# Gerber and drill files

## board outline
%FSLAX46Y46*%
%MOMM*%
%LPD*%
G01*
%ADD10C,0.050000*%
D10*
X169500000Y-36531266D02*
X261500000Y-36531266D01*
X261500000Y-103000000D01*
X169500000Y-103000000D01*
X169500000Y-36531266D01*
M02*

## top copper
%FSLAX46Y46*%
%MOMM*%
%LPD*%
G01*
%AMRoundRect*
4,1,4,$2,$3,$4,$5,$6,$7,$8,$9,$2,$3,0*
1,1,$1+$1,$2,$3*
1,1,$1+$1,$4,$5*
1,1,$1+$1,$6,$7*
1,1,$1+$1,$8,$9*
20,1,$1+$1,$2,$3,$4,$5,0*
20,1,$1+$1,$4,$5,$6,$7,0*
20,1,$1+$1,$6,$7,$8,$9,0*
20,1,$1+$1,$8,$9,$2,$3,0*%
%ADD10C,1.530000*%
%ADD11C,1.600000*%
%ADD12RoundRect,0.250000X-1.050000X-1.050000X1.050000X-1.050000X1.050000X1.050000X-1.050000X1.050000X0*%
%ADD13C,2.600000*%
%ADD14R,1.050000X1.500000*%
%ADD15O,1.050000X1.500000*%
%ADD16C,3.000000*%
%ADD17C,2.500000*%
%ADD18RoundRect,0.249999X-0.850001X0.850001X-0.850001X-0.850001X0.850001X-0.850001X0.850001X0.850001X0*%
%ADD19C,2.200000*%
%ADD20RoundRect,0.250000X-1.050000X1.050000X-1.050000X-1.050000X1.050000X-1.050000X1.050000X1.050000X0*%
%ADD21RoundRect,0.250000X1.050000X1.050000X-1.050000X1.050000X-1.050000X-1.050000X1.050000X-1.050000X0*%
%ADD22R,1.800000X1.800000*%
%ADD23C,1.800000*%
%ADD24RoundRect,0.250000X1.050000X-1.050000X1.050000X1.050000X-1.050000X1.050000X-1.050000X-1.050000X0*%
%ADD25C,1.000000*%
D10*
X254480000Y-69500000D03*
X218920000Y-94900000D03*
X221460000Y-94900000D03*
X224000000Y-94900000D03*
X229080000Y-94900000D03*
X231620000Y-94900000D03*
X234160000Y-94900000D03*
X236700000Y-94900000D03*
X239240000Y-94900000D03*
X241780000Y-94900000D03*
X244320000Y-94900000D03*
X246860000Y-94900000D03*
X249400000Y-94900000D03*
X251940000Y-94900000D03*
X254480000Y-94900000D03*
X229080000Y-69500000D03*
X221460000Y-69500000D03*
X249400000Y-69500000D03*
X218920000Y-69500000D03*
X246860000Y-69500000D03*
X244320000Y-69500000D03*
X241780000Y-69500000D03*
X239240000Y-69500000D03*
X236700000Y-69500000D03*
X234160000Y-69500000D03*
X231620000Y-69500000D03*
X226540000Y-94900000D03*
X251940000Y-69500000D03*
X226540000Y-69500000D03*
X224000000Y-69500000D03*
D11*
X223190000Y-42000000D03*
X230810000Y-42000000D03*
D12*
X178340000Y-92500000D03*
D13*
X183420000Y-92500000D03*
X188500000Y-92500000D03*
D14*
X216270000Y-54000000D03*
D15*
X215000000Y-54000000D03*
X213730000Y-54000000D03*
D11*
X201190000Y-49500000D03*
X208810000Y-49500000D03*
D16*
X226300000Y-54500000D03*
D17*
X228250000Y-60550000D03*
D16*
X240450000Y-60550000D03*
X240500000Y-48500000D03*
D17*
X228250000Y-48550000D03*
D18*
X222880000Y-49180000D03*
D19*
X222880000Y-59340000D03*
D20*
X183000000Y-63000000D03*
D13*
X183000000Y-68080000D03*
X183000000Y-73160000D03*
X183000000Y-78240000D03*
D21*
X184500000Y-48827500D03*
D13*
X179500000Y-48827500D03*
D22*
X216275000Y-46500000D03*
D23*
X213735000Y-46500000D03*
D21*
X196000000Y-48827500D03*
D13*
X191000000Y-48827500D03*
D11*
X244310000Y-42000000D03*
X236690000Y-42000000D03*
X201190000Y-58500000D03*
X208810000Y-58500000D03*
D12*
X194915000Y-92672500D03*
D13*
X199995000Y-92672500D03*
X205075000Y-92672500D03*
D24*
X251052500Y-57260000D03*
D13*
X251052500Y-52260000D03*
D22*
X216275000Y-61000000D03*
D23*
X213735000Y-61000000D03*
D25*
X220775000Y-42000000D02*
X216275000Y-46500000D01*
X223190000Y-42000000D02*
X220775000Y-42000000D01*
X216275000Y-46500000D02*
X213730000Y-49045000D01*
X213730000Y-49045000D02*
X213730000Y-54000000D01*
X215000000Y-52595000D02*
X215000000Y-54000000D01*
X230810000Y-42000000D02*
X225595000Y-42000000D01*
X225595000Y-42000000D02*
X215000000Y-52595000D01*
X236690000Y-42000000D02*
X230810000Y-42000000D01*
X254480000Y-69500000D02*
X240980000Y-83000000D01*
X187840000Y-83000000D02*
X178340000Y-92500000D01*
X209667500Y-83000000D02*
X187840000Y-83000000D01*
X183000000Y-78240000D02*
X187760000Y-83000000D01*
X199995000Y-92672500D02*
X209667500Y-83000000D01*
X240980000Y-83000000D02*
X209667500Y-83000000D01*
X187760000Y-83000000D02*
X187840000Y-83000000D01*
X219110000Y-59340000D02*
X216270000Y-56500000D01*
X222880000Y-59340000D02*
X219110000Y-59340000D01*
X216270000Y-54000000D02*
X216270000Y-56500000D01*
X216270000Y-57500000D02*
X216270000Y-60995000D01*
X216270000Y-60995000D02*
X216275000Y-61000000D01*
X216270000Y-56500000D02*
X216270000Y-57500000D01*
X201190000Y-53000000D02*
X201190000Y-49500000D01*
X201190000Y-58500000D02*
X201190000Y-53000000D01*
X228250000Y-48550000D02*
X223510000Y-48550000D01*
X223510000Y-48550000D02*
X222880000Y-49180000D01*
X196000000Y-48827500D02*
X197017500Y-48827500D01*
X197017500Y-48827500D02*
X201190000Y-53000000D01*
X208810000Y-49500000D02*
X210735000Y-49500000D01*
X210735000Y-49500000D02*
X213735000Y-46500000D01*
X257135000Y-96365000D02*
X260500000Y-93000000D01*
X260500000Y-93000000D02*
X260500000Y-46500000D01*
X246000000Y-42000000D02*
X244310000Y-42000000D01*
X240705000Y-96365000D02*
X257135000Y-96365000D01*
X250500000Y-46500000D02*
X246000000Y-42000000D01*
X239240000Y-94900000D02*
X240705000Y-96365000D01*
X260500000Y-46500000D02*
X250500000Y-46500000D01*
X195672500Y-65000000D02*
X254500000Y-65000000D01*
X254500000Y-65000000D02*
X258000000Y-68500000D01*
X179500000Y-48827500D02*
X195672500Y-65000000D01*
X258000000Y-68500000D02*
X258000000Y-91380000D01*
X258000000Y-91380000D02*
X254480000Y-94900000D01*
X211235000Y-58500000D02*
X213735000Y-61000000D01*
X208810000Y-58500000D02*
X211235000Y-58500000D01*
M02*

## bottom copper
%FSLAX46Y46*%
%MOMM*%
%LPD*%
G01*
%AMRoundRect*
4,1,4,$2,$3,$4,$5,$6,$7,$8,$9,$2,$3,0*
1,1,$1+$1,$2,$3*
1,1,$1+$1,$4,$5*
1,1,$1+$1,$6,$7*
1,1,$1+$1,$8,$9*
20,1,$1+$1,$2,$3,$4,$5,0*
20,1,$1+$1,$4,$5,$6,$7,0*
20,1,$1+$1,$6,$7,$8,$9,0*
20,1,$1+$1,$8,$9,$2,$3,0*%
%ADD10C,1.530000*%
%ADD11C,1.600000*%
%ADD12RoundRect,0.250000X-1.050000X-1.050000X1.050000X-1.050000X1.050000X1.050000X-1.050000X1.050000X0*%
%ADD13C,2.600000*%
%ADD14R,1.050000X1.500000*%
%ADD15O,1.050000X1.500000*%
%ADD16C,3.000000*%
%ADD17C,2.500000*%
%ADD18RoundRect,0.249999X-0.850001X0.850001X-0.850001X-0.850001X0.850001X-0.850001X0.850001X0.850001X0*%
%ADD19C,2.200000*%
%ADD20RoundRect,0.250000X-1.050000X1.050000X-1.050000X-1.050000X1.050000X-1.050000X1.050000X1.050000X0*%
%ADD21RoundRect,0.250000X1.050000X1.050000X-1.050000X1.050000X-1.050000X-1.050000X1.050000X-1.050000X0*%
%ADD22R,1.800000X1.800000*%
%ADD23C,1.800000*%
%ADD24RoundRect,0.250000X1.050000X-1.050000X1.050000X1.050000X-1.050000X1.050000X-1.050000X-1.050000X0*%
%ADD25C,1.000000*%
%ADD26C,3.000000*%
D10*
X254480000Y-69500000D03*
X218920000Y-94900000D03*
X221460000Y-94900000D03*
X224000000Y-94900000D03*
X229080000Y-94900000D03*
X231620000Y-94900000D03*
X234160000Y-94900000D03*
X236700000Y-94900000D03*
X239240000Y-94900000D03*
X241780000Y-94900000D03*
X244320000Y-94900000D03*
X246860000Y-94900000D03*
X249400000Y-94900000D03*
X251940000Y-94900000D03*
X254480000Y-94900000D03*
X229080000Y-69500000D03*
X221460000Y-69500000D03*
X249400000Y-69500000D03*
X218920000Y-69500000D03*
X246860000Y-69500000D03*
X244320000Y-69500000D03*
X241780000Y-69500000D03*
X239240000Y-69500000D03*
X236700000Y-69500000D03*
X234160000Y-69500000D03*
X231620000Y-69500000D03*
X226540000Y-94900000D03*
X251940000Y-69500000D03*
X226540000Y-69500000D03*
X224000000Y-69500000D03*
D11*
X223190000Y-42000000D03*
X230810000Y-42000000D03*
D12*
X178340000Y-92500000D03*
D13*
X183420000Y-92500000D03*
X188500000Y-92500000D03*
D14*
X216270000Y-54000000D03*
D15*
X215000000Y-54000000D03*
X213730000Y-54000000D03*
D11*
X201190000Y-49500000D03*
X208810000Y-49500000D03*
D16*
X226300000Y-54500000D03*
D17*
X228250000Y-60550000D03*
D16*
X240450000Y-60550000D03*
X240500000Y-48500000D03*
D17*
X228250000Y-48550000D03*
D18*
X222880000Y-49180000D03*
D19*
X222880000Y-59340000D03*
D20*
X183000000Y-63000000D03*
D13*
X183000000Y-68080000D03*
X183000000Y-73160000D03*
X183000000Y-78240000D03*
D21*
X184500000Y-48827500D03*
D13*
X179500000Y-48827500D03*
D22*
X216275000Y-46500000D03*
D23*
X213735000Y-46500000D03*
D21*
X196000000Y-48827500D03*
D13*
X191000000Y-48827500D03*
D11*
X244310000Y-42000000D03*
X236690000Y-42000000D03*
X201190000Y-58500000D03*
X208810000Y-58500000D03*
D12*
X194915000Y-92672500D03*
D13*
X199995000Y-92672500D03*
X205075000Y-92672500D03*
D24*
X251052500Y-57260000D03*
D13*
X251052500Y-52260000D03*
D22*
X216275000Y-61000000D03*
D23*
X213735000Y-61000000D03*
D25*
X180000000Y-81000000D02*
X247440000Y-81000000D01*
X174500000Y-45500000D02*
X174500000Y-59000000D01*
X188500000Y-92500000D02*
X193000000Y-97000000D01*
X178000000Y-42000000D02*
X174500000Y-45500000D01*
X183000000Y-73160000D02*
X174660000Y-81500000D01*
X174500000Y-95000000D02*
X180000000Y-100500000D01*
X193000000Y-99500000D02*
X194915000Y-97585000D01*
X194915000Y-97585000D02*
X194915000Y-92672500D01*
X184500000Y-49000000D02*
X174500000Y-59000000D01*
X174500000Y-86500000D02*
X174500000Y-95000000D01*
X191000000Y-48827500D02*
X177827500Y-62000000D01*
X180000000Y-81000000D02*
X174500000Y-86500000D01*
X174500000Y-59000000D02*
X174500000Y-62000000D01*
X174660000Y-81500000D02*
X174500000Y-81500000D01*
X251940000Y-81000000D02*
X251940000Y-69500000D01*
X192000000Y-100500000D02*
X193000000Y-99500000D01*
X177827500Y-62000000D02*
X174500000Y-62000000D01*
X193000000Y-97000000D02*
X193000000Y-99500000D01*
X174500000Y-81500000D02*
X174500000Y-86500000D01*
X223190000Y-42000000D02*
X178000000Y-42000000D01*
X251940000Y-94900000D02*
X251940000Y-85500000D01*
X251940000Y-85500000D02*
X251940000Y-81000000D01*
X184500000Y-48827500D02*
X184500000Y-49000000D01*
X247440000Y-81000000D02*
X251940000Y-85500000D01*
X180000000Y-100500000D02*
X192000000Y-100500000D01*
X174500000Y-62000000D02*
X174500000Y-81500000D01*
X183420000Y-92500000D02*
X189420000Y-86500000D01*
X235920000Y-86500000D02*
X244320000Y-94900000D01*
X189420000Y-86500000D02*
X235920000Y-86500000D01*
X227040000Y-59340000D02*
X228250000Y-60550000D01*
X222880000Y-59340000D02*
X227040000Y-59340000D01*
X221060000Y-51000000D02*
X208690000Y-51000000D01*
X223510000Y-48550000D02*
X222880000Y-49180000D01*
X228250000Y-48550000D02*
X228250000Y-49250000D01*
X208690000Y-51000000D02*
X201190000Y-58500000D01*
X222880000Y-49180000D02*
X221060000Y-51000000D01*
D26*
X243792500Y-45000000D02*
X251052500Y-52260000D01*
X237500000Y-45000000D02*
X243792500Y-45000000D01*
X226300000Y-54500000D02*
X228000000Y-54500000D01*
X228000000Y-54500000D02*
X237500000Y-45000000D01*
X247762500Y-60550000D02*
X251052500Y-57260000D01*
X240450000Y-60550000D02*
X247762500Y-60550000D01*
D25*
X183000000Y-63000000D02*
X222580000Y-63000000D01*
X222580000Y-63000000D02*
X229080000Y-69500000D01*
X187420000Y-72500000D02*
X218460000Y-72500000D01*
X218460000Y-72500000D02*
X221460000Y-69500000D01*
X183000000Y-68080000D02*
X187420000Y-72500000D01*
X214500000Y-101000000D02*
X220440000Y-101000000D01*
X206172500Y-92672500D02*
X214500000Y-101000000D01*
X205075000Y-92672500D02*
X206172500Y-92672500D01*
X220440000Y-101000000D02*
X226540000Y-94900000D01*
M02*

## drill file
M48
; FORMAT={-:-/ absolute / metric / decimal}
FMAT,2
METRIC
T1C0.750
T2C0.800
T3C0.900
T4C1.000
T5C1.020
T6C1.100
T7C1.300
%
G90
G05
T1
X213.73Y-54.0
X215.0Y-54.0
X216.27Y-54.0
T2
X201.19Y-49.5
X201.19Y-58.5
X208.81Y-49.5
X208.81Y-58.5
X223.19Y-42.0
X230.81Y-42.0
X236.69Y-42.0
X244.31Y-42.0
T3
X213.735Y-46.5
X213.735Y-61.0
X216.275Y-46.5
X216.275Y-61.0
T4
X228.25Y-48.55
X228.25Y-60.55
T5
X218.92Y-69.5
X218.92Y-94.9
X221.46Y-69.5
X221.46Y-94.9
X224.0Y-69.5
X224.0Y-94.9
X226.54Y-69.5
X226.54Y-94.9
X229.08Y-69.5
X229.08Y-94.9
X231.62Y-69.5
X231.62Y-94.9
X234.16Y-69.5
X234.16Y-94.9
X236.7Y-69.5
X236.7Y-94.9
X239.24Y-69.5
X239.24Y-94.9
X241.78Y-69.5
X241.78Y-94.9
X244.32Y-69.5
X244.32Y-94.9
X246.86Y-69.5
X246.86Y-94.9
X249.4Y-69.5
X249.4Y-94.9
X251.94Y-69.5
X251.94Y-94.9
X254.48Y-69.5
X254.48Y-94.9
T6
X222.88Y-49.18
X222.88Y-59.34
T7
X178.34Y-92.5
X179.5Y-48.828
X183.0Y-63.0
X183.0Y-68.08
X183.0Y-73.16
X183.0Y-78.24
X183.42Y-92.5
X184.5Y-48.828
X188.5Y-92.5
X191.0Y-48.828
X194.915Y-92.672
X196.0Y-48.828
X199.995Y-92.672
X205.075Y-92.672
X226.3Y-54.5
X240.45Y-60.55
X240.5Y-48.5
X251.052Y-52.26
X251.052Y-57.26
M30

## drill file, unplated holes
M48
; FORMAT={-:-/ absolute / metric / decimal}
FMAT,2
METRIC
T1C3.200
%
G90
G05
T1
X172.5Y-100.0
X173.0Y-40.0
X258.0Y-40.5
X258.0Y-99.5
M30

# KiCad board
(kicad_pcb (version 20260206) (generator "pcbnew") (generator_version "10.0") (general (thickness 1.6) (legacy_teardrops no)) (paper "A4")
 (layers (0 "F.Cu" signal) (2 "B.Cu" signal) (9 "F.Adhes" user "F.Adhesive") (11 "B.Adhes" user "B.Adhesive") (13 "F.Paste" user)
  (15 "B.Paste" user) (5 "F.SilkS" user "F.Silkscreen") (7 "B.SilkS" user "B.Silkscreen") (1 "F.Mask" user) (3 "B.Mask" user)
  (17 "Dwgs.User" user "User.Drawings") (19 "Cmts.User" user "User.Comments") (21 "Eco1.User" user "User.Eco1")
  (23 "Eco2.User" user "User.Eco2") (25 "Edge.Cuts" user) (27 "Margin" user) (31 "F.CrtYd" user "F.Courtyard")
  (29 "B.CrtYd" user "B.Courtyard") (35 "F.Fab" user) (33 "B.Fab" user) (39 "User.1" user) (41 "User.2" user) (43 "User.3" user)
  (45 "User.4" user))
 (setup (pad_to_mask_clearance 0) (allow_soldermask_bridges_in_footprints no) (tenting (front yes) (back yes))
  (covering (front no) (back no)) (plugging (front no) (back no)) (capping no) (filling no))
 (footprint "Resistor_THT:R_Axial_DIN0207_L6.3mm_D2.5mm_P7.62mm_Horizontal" (layer "F.Cu") (at 223.19 42)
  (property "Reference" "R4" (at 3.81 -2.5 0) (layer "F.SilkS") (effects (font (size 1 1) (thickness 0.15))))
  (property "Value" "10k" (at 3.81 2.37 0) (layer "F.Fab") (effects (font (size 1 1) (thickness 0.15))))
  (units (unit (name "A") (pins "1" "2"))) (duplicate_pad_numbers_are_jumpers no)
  (pad "1" thru_hole circle (at 0 0) (size 1.6 1.6) (drill 0.8) (layers "*.Cu" "*.Mask") (remove_unused_layers no) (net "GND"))
  (pad "2" thru_hole circle (at 7.62 0) (size 1.6 1.6) (drill 0.8) (layers "*.Cu" "*.Mask") (remove_unused_layers no) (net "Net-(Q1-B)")))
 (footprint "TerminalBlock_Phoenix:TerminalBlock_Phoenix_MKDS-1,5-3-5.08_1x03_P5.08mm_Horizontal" (layer "F.Cu") (at 178.34 92.5)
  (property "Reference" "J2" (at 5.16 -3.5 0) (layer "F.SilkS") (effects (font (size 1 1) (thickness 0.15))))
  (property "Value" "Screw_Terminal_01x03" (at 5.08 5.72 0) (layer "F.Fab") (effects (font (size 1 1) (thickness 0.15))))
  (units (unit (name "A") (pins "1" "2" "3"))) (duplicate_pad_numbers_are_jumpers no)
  (pad "1" thru_hole roundrect (at 0 0) (size 2.6 2.6) (drill 1.3) (layers "*.Cu" "*.Mask") (remove_unused_layers no)
   (roundrect_rratio 0.096154) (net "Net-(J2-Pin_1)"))
  (pad "2" thru_hole circle (at 5.08 0) (size 2.6 2.6) (drill 1.3) (layers "*.Cu" "*.Mask") (remove_unused_layers no) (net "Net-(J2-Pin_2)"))
  (pad "3" thru_hole circle (at 10.16 0) (size 2.6 2.6) (drill 1.3) (layers "*.Cu" "*.Mask") (remove_unused_layers no) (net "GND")))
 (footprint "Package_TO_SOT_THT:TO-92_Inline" (layer "F.Cu") (at 216.27 54 180)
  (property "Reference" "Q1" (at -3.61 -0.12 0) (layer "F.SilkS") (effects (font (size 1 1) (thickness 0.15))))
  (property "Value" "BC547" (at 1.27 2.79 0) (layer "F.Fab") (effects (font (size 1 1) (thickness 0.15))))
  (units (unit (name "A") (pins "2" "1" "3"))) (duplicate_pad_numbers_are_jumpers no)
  (pad "1" thru_hole rect (at 0 0 180) (size 1.05 1.5) (drill 0.75) (layers "*.Cu" "*.Mask") (remove_unused_layers no) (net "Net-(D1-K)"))
  (pad "2" thru_hole oval (at 1.27 0 180) (size 1.05 1.5) (drill 0.75) (layers "*.Cu" "*.Mask") (remove_unused_layers no) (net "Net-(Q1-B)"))
  (pad "3" thru_hole oval (at 2.54 0 180) (size 1.05 1.5) (drill 0.75) (layers "*.Cu" "*.Mask") (remove_unused_layers no) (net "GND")))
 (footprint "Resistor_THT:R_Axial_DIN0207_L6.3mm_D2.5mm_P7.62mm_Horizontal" (layer "F.Cu") (at 201.19 49.5)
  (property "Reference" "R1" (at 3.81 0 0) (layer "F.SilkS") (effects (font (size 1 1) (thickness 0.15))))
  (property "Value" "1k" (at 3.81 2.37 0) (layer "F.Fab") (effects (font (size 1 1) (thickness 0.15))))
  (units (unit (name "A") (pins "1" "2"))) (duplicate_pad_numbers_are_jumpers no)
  (pad "1" thru_hole circle (at 0 0) (size 1.6 1.6) (drill 0.8) (layers "*.Cu" "*.Mask") (remove_unused_layers no) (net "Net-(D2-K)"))
  (pad "2" thru_hole circle (at 7.62 0) (size 1.6 1.6) (drill 0.8) (layers "*.Cu" "*.Mask") (remove_unused_layers no) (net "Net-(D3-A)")))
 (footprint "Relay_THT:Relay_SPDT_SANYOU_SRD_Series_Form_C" (layer "F.Cu") (at 226.3 54.5)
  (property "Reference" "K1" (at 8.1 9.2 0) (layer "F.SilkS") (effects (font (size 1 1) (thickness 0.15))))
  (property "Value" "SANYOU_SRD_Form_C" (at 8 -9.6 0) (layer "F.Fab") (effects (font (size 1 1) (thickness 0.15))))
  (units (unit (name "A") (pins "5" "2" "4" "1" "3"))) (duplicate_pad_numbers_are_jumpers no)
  (pad "1" thru_hole circle (at 0 0 90) (size 3 3) (drill 1.3) (layers "*.Cu" "*.Mask") (remove_unused_layers no) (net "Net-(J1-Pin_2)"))
  (pad "2" thru_hole circle (at 1.95 6.05 90) (size 2.5 2.5) (drill 1) (layers "*.Cu" "*.Mask") (remove_unused_layers no) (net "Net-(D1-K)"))
  (pad "3" thru_hole circle (at 14.15 6.05 90) (size 3 3) (drill 1.3) (layers "*.Cu" "*.Mask") (remove_unused_layers no)
   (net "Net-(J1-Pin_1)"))
  (pad "4" thru_hole circle (at 14.2 -6 90) (size 3 3) (drill 1.3) (layers "*.Cu" "*.Mask") (remove_unused_layers no)
   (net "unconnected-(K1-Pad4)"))
  (pad "5" thru_hole circle (at 1.95 -5.95 90) (size 2.5 2.5) (drill 1) (layers "*.Cu" "*.Mask") (remove_unused_layers no)
   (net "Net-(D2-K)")))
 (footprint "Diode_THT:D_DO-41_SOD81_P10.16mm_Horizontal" (layer "F.Cu") (at 222.88 49.18 -90)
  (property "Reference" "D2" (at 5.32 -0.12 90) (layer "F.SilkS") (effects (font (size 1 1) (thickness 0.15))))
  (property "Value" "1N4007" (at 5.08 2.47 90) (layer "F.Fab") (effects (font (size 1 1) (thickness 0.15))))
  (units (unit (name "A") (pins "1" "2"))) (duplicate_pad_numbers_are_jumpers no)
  (pad "1" thru_hole roundrect (at 0 0 270) (size 2.2 2.2) (drill 1.1) (layers "*.Cu" "*.Mask") (remove_unused_layers no)
   (roundrect_rratio 0.113636) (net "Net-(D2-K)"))
  (pad "2" thru_hole circle (at 10.16 0 270) (size 2.2 2.2) (drill 1.1) (layers "*.Cu" "*.Mask") (remove_unused_layers no)
   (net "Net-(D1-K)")))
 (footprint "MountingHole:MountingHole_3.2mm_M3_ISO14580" (layer "F.Cu") (at 258 40.5)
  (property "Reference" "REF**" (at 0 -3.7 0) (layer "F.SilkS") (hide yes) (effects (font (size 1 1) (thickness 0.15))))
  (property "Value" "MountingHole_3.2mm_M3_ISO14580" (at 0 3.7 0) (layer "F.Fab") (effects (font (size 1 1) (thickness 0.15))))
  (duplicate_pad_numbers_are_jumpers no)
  (pad "" np_thru_hole circle (at 0 0) (size 3.2 3.2) (drill 3.2) (layers "*.Cu" "*.Mask")))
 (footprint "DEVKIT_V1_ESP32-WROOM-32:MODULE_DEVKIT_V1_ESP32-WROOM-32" (layer "F.Cu") (at 231.61 82.2 90)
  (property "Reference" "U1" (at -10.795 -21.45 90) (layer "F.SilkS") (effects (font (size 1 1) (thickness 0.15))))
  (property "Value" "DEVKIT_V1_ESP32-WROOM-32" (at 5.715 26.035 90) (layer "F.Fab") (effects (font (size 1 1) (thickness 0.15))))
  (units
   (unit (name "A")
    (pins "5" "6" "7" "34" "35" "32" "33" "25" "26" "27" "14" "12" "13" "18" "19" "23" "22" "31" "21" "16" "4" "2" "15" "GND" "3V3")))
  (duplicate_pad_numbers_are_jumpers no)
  (pad "3V3" thru_hole circle (at 12.7 22.87 90) (size 1.53 1.53) (drill 1.02) (layers "*.Cu" "*.Mask") (remove_unused_layers no)
   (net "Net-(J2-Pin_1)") (solder_mask_margin 0.102))
  (pad "5" thru_hole circle (at -12.7 -12.69 90) (size 1.53 1.53) (drill 1.02) (layers "*.Cu" "*.Mask") (remove_unused_layers no)
   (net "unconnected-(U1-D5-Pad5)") (solder_mask_margin 0.102))
  (pad "6" thru_hole circle (at -12.7 -10.15 90) (size 1.53 1.53) (drill 1.02) (layers "*.Cu" "*.Mask") (remove_unused_layers no)
   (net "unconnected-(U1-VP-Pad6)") (solder_mask_margin 0.102))
  (pad "7" thru_hole circle (at -12.7 -7.61 90) (size 1.53 1.53) (drill 1.02) (layers "*.Cu" "*.Mask") (remove_unused_layers no)
   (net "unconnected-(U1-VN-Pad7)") (solder_mask_margin 0.102))
  (pad "9" thru_hole circle (at -12.7 -2.53 90) (size 1.53 1.53) (drill 1.02) (layers "*.Cu" "*.Mask") (remove_unused_layers no)
   (solder_mask_margin 0.102))
  (pad "10" thru_hole circle (at -12.7 0.01 90) (size 1.53 1.53) (drill 1.02) (layers "*.Cu" "*.Mask") (remove_unused_layers no)
   (solder_mask_margin 0.102))
  (pad "11" thru_hole circle (at -12.7 2.55 90) (size 1.53 1.53) (drill 1.02) (layers "*.Cu" "*.Mask") (remove_unused_layers no)
   (solder_mask_margin 0.102))
  (pad "12" thru_hole circle (at -12.7 5.09 90) (size 1.53 1.53) (drill 1.02) (layers "*.Cu" "*.Mask") (remove_unused_layers no)
   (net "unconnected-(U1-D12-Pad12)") (solder_mask_margin 0.102))
  (pad "13" thru_hole circle (at -12.7 7.63 90) (size 1.53 1.53) (drill 1.02) (layers "*.Cu" "*.Mask") (remove_unused_layers no)
   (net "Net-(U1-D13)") (solder_mask_margin 0.102))
  (pad "14" thru_hole circle (at -12.7 10.17 90) (size 1.53 1.53) (drill 1.02) (layers "*.Cu" "*.Mask") (remove_unused_layers no)
   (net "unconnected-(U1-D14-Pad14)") (solder_mask_margin 0.102))
  (pad "15" thru_hole circle (at -12.7 12.71 90) (size 1.53 1.53) (drill 1.02) (layers "*.Cu" "*.Mask") (remove_unused_layers no)
   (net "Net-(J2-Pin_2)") (solder_mask_margin 0.102))
  (pad "16" thru_hole circle (at -12.7 15.25 90) (size 1.53 1.53) (drill 1.02) (layers "*.Cu" "*.Mask") (remove_unused_layers no)
   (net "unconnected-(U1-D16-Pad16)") (solder_mask_margin 0.102))
  (pad "17" thru_hole circle (at -12.7 17.79 90) (size 1.53 1.53) (drill 1.02) (layers "*.Cu" "*.Mask") (remove_unused_layers no)
   (solder_mask_margin 0.102))
  (pad "18" thru_hole circle (at -12.7 20.33 90) (size 1.53 1.53) (drill 1.02) (layers "*.Cu" "*.Mask") (remove_unused_layers no)
   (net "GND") (solder_mask_margin 0.102))
  (pad "19" thru_hole circle (at -12.7 22.87 90) (size 1.53 1.53) (drill 1.02) (layers "*.Cu" "*.Mask") (remove_unused_layers no)
   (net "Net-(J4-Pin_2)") (solder_mask_margin 0.102))
  (pad "21" thru_hole circle (at 12.7 -2.53 90) (size 1.53 1.53) (drill 1.02) (layers "*.Cu" "*.Mask") (remove_unused_layers no)
   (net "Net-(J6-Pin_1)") (solder_mask_margin 0.102))
  (pad "22" thru_hole circle (at 12.7 -10.15 90) (size 1.53 1.53) (drill 1.02) (layers "*.Cu" "*.Mask") (remove_unused_layers no)
   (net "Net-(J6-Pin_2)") (solder_mask_margin 0.102))
  (pad "22" thru_hole circle (at 12.7 17.79 90) (size 1.53 1.53) (drill 1.02) (layers "*.Cu" "*.Mask") (remove_unused_layers no)
   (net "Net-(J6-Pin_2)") (solder_mask_margin 0.102))
  (pad "23" thru_hole circle (at 12.7 -12.69 90) (size 1.53 1.53) (drill 1.02) (layers "*.Cu" "*.Mask") (remove_unused_layers no)
   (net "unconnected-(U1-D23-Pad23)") (solder_mask_margin 0.102))
  (pad "23" thru_hole circle (at 12.7 15.25 90) (size 1.53 1.53) (drill 1.02) (layers "*.Cu" "*.Mask") (remove_unused_layers no)
   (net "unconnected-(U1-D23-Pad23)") (solder_mask_margin 0.102))
  (pad "24" thru_hole circle (at 12.7 12.71 90) (size 1.53 1.53) (drill 1.02) (layers "*.Cu" "*.Mask") (remove_unused_layers no)
   (solder_mask_margin 0.102))
  (pad "25" thru_hole circle (at 12.7 10.17 90) (size 1.53 1.53) (drill 1.02) (layers "*.Cu" "*.Mask") (remove_unused_layers no)
   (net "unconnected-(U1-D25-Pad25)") (solder_mask_margin 0.102))
  (pad "26" thru_hole circle (at 12.7 7.63 90) (size 1.53 1.53) (drill 1.02) (layers "*.Cu" "*.Mask") (remove_unused_layers no)
   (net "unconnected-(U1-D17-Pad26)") (solder_mask_margin 0.102))
  (pad "27" thru_hole circle (at 12.7 5.09 90) (size 1.53 1.53) (drill 1.02) (layers "*.Cu" "*.Mask") (remove_unused_layers no)
   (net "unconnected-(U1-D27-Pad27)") (solder_mask_margin 0.102))
  (pad "28" thru_hole circle (at 12.7 2.55 90) (size 1.53 1.53) (drill 1.02) (layers "*.Cu" "*.Mask") (remove_unused_layers no)
   (solder_mask_margin 0.102))
  (pad "29" thru_hole circle (at 12.7 0.01 90) (size 1.53 1.53) (drill 1.02) (layers "*.Cu" "*.Mask") (remove_unused_layers no)
   (solder_mask_margin 0.102))
  (pad "34" thru_hole circle (at -12.7 -5.07 90) (size 1.53 1.53) (drill 1.02) (layers "*.Cu" "*.Mask") (remove_unused_layers no)
   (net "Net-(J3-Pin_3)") (solder_mask_margin 0.102))
  (pad "GND" thru_hole circle (at 12.7 20.33 90) (size 1.53 1.53) (drill 1.02) (layers "*.Cu" "*.Mask") (remove_unused_layers no)
   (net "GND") (solder_mask_margin 0.102))
  (pad "RX0" thru_hole circle (at 12.7 -5.07 90) (size 1.53 1.53) (drill 1.02) (layers "*.Cu" "*.Mask") (remove_unused_layers no)
   (solder_mask_margin 0.102))
  (pad "TX0" thru_hole circle (at 12.7 -7.61 90) (size 1.53 1.53) (drill 1.02) (layers "*.Cu" "*.Mask") (remove_unused_layers no)
   (solder_mask_margin 0.102)))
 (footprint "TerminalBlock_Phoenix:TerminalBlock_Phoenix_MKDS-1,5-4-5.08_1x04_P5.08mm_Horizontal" (layer "F.Cu") (at 183 63 -90)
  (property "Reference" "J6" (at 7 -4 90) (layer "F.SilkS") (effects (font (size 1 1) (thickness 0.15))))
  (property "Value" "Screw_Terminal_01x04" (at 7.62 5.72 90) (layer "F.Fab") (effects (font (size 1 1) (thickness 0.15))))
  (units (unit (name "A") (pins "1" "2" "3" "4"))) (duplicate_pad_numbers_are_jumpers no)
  (pad "1" thru_hole roundrect (at 0 0 270) (size 2.6 2.6) (drill 1.3) (layers "*.Cu" "*.Mask") (remove_unused_layers no)
   (roundrect_rratio 0.096154) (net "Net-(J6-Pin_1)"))
  (pad "2" thru_hole circle (at 5.08 0 270) (size 2.6 2.6) (drill 1.3) (layers "*.Cu" "*.Mask") (remove_unused_layers no)
   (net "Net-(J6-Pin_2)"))
  (pad "3" thru_hole circle (at 10.16 0 270) (size 2.6 2.6) (drill 1.3) (layers "*.Cu" "*.Mask") (remove_unused_layers no) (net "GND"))
  (pad "4" thru_hole circle (at 15.24 0 270) (size 2.6 2.6) (drill 1.3) (layers "*.Cu" "*.Mask") (remove_unused_layers no)
   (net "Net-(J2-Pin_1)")))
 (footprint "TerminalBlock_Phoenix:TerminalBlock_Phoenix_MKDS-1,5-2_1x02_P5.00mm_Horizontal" (layer "F.Cu") (at 184.5 48.8275 180)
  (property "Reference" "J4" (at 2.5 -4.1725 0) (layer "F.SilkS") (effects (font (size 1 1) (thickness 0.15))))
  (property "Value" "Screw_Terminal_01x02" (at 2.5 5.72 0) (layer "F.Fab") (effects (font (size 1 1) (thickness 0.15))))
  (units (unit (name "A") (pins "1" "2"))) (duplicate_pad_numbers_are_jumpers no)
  (pad "1" thru_hole roundrect (at 0 0 180) (size 2.6 2.6) (drill 1.3) (layers "*.Cu" "*.Mask") (remove_unused_layers no)
   (roundrect_rratio 0.096154) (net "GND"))
  (pad "2" thru_hole circle (at 5 0 180) (size 2.6 2.6) (drill 1.3) (layers "*.Cu" "*.Mask") (remove_unused_layers no)
   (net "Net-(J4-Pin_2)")))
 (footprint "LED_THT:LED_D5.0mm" (layer "F.Cu") (at 216.275 46.5 180)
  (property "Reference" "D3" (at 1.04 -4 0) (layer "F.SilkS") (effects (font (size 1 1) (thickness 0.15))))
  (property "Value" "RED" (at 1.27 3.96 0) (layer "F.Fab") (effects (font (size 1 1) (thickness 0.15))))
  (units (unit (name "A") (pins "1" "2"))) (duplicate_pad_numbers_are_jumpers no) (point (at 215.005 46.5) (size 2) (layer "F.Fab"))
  (pad "1" thru_hole rect (at 0 0 180) (size 1.8 1.8) (drill 0.9) (layers "*.Cu" "*.Mask") (remove_unused_layers no) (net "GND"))
  (pad "2" thru_hole circle (at 2.54 0 180) (size 1.8 1.8) (drill 0.9) (layers "*.Cu" "*.Mask") (remove_unused_layers no) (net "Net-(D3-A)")))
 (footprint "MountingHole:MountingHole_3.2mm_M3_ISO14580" (layer "F.Cu") (at 258 99.5)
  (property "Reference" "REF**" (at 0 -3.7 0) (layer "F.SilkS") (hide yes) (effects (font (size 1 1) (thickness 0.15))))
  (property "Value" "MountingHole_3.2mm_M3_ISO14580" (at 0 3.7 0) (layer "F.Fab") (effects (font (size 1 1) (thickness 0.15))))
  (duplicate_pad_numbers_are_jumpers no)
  (pad "" np_thru_hole circle (at 0 0) (size 3.2 3.2) (drill 3.2) (layers "*.Cu" "*.Mask")))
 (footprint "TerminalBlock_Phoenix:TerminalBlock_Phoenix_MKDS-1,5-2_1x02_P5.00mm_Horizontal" (layer "F.Cu") (at 196 48.8275 180)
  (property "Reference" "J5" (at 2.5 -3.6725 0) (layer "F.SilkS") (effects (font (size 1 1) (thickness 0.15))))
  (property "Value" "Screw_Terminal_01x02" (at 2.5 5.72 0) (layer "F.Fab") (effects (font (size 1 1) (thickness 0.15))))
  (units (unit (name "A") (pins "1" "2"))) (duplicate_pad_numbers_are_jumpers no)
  (pad "1" thru_hole roundrect (at 0 0 180) (size 2.6 2.6) (drill 1.3) (layers "*.Cu" "*.Mask") (remove_unused_layers no)
   (roundrect_rratio 0.096154) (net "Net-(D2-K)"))
  (pad "2" thru_hole circle (at 5 0 180) (size 2.6 2.6) (drill 1.3) (layers "*.Cu" "*.Mask") (remove_unused_layers no) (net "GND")))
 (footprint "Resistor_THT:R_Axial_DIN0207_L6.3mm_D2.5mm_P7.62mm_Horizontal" (layer "F.Cu") (at 244.31 42 180)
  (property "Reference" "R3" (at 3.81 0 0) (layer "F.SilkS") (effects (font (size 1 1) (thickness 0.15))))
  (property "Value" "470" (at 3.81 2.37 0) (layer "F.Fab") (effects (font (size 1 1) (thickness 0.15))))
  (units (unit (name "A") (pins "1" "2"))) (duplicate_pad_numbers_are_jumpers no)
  (pad "1" thru_hole circle (at 0 0 180) (size 1.6 1.6) (drill 0.8) (layers "*.Cu" "*.Mask") (remove_unused_layers no) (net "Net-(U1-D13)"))
  (pad "2" thru_hole circle (at 7.62 0 180) (size 1.6 1.6) (drill 0.8) (layers "*.Cu" "*.Mask") (remove_unused_layers no) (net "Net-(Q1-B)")))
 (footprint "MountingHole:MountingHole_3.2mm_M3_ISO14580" (layer "F.Cu") (at 173 40)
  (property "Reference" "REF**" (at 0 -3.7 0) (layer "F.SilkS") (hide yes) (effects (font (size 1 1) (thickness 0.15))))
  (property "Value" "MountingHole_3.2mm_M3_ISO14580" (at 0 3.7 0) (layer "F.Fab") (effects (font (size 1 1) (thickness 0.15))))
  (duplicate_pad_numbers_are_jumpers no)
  (pad "" np_thru_hole circle (at 0 0) (size 3.2 3.2) (drill 3.2) (layers "*.Cu" "*.Mask")))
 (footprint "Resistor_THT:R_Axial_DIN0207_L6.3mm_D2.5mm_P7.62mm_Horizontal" (layer "F.Cu") (at 201.19 58.5)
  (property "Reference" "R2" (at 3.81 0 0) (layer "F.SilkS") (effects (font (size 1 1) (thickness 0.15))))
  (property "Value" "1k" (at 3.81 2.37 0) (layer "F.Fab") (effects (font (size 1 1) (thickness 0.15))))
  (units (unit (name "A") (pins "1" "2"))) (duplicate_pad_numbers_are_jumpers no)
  (pad "1" thru_hole circle (at 0 0) (size 1.6 1.6) (drill 0.8) (layers "*.Cu" "*.Mask") (remove_unused_layers no) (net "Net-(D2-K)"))
  (pad "2" thru_hole circle (at 7.62 0) (size 1.6 1.6) (drill 0.8) (layers "*.Cu" "*.Mask") (remove_unused_layers no) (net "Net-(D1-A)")))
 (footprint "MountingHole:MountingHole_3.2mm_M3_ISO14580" (layer "F.Cu") (at 172.5 100)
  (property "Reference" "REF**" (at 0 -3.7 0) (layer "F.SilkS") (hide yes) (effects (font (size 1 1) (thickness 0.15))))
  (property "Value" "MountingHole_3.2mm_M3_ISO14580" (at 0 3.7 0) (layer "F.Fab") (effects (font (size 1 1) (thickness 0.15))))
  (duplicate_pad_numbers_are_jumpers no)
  (pad "" np_thru_hole circle (at 0 0) (size 3.2 3.2) (drill 3.2) (layers "*.Cu" "*.Mask")))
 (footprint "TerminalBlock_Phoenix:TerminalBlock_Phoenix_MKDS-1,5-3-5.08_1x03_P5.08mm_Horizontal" (layer "F.Cu") (at 194.915 92.6725)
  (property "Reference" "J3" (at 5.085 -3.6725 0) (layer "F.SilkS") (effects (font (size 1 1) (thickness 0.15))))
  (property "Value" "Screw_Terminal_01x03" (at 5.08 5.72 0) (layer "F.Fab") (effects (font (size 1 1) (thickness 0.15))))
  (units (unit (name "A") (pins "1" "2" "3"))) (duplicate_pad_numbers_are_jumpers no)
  (pad "1" thru_hole roundrect (at 0 0) (size 2.6 2.6) (drill 1.3) (layers "*.Cu" "*.Mask") (remove_unused_layers no)
   (roundrect_rratio 0.096154) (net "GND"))
  (pad "2" thru_hole circle (at 5.08 0) (size 2.6 2.6) (drill 1.3) (layers "*.Cu" "*.Mask") (remove_unused_layers no) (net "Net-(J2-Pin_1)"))
  (pad "3" thru_hole circle (at 10.16 0) (size 2.6 2.6) (drill 1.3) (layers "*.Cu" "*.Mask") (remove_unused_layers no)
   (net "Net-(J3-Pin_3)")))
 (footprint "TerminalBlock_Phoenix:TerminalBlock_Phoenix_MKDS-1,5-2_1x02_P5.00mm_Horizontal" (layer "F.Cu") (at 251.0525 57.26 90)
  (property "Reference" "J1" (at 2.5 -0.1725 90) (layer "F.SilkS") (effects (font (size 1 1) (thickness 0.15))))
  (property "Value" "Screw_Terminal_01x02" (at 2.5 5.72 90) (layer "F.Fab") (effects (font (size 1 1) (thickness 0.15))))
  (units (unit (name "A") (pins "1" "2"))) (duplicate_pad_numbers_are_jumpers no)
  (pad "1" thru_hole roundrect (at 0 0 90) (size 2.6 2.6) (drill 1.3) (layers "*.Cu" "*.Mask") (remove_unused_layers no)
   (roundrect_rratio 0.096154) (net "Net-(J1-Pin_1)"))
  (pad "2" thru_hole circle (at 5 0 90) (size 2.6 2.6) (drill 1.3) (layers "*.Cu" "*.Mask") (remove_unused_layers no) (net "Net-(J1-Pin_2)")))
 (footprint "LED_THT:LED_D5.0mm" (layer "F.Cu") (at 216.275 61 180)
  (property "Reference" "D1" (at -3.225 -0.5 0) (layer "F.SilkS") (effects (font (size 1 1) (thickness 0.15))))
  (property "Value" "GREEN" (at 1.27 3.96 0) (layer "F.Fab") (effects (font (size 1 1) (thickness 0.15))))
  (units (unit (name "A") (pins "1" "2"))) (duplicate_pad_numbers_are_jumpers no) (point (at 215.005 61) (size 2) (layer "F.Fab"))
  (pad "1" thru_hole rect (at 0 0 180) (size 1.8 1.8) (drill 0.9) (layers "*.Cu" "*.Mask") (remove_unused_layers no) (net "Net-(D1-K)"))
  (pad "2" thru_hole circle (at 2.54 0 180) (size 1.8 1.8) (drill 0.9) (layers "*.Cu" "*.Mask") (remove_unused_layers no) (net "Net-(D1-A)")))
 (gr_rect (start 169.5 36.531266) (end 261.5 103) (stroke (width 0.05) (type default)) (fill no) (layer "Edge.Cuts"))
 (segment (start 220.775 42) (end 216.275 46.5) (width 1) (layer "F.Cu") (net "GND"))
 (segment (start 223.19 42) (end 220.775 42) (width 1) (layer "F.Cu") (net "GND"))
 (segment (start 216.275 46.5) (end 213.73 49.045) (width 1) (layer "F.Cu") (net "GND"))
 (segment (start 213.73 49.045) (end 213.73 54) (width 1) (layer "F.Cu") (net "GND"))
 (segment (start 180 81) (end 247.44 81) (width 1) (layer "B.Cu") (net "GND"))
 (segment (start 174.5 45.5) (end 174.5 59) (width 1) (layer "B.Cu") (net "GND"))
 (segment (start 188.5 92.5) (end 193 97) (width 1) (layer "B.Cu") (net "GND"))
 (segment (start 178 42) (end 174.5 45.5) (width 1) (layer "B.Cu") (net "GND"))
 (segment (start 183 73.16) (end 174.66 81.5) (width 1) (layer "B.Cu") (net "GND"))
 (segment (start 174.5 95) (end 180 100.5) (width 1) (layer "B.Cu") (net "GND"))
 (segment (start 193 99.5) (end 194.915 97.585) (width 1) (layer "B.Cu") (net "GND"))
 (segment (start 194.915 97.585) (end 194.915 92.6725) (width 1) (layer "B.Cu") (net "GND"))
 (segment (start 184.5 49) (end 174.5 59) (width 1) (layer "B.Cu") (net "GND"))
 (segment (start 174.5 86.5) (end 174.5 95) (width 1) (layer "B.Cu") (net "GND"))
 (segment (start 191 48.8275) (end 177.8275 62) (width 1) (layer "B.Cu") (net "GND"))
 (segment (start 180 81) (end 174.5 86.5) (width 1) (layer "B.Cu") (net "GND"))
 (segment (start 174.5 59) (end 174.5 62) (width 1) (layer "B.Cu") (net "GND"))
 (segment (start 174.66 81.5) (end 174.5 81.5) (width 1) (layer "B.Cu") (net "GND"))
 (segment (start 251.94 81) (end 251.94 69.5) (width 1) (layer "B.Cu") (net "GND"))
 (segment (start 192 100.5) (end 193 99.5) (width 1) (layer "B.Cu") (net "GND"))
 (segment (start 177.8275 62) (end 174.5 62) (width 1) (layer "B.Cu") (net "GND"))
 (segment (start 193 97) (end 193 99.5) (width 1) (layer "B.Cu") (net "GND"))
 (segment (start 174.5 81.5) (end 174.5 86.5) (width 1) (layer "B.Cu") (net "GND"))
 (segment (start 223.19 42) (end 178 42) (width 1) (layer "B.Cu") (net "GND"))
 (segment (start 251.94 94.9) (end 251.94 85.5) (width 1) (layer "B.Cu") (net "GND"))
 (segment (start 251.94 85.5) (end 251.94 81) (width 1) (layer "B.Cu") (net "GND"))
 (segment (start 184.5 48.8275) (end 184.5 49) (width 1) (layer "B.Cu") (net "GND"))
 (segment (start 247.44 81) (end 251.94 85.5) (width 1) (layer "B.Cu") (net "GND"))
 (segment (start 180 100.5) (end 192 100.5) (width 1) (layer "B.Cu") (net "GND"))
 (segment (start 174.5 62) (end 174.5 81.5) (width 1) (layer "B.Cu") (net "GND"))
 (segment (start 215 52.595) (end 215 54) (width 1) (layer "F.Cu") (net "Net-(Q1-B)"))
 (segment (start 230.81 42) (end 225.595 42) (width 1) (layer "F.Cu") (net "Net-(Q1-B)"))
 (segment (start 225.595 42) (end 215 52.595) (width 1) (layer "F.Cu") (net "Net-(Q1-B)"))
 (segment (start 236.69 42) (end 230.81 42) (width 1) (layer "F.Cu") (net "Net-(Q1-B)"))
 (segment (start 254.48 69.5) (end 240.98 83) (width 1) (layer "F.Cu") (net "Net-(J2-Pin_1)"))
 (segment (start 187.84 83) (end 178.34 92.5) (width 1) (layer "F.Cu") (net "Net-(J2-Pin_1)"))
 (segment (start 209.6675 83) (end 187.84 83) (width 1) (layer "F.Cu") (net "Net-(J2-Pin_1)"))
 (segment (start 183 78.24) (end 187.76 83) (width 1) (layer "F.Cu") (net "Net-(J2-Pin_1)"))
 (segment (start 199.995 92.6725) (end 209.6675 83) (width 1) (layer "F.Cu") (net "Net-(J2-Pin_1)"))
 (segment (start 240.98 83) (end 209.6675 83) (width 1) (layer "F.Cu") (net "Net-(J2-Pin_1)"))
 (segment (start 187.76 83) (end 187.84 83) (width 1) (layer "F.Cu") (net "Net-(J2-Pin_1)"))
 (segment (start 183.42 92.5) (end 189.42 86.5) (width 1) (layer "B.Cu") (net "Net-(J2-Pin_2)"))
 (segment (start 235.92 86.5) (end 244.32 94.9) (width 1) (layer "B.Cu") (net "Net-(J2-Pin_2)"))
 (segment (start 189.42 86.5) (end 235.92 86.5) (width 1) (layer "B.Cu") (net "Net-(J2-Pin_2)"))
 (segment (start 219.11 59.34) (end 216.27 56.5) (width 1) (layer "F.Cu") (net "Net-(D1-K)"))
 (segment (start 222.88 59.34) (end 219.11 59.34) (width 1) (layer "F.Cu") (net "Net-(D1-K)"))
 (segment (start 216.27 54) (end 216.27 56.5) (width 1) (layer "F.Cu") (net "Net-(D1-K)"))
 (segment (start 216.27 57.5) (end 216.27 60.995) (width 1) (layer "F.Cu") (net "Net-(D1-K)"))
 (segment (start 216.27 60.995) (end 216.275 61) (width 1) (layer "F.Cu") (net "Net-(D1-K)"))
 (segment (start 216.27 56.5) (end 216.27 57.5) (width 1) (layer "F.Cu") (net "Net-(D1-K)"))
 (segment (start 227.04 59.34) (end 228.25 60.55) (width 1) (layer "B.Cu") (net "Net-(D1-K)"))
 (segment (start 222.88 59.34) (end 227.04 59.34) (width 1) (layer "B.Cu") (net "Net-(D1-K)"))
 (segment (start 201.19 53) (end 201.19 49.5) (width 1) (layer "F.Cu") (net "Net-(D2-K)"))
 (segment (start 201.19 58.5) (end 201.19 53) (width 1) (layer "F.Cu") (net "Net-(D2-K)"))
 (segment (start 228.25 48.55) (end 223.51 48.55) (width 1) (layer "F.Cu") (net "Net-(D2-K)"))
 (segment (start 223.51 48.55) (end 222.88 49.18) (width 1) (layer "F.Cu") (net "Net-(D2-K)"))
 (segment (start 196 48.8275) (end 197.0175 48.8275) (width 1) (layer "F.Cu") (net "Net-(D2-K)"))
 (segment (start 197.0175 48.8275) (end 201.19 53) (width 1) (layer "F.Cu") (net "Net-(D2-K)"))
 (segment (start 221.06 51) (end 208.69 51) (width 1) (layer "B.Cu") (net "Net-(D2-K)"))
 (segment (start 223.51 48.55) (end 222.88 49.18) (width 1) (layer "B.Cu") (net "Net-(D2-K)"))
 (segment (start 228.25 48.55) (end 228.25 49.25) (width 1) (layer "B.Cu") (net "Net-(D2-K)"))
 (segment (start 208.69 51) (end 201.19 58.5) (width 1) (layer "B.Cu") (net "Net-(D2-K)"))
 (segment (start 222.88 49.18) (end 221.06 51) (width 1) (layer "B.Cu") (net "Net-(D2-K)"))
 (segment (start 208.81 49.5) (end 210.735 49.5) (width 1) (layer "F.Cu") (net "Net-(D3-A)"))
 (segment (start 210.735 49.5) (end 213.735 46.5) (width 1) (layer "F.Cu") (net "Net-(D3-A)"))
 (segment (start 243.7925 45) (end 251.0525 52.26) (width 3) (layer "B.Cu") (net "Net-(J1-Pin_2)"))
 (segment (start 237.5 45) (end 243.7925 45) (width 3) (layer "B.Cu") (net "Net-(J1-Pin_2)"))
 (segment (start 226.3 54.5) (end 228 54.5) (width 3) (layer "B.Cu") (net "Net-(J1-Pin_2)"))
 (segment (start 228 54.5) (end 237.5 45) (width 3) (layer "B.Cu") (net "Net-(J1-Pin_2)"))
 (segment (start 247.7625 60.55) (end 251.0525 57.26) (width 3) (layer "B.Cu") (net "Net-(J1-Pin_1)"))
 (segment (start 240.45 60.55) (end 247.7625 60.55) (width 3) (layer "B.Cu") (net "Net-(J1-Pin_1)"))
 (segment (start 257.135 96.365) (end 260.5 93) (width 1) (layer "F.Cu") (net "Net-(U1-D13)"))
 (segment (start 260.5 93) (end 260.5 46.5) (width 1) (layer "F.Cu") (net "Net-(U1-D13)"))
 (segment (start 246 42) (end 244.31 42) (width 1) (layer "F.Cu") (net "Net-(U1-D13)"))
 (segment (start 240.705 96.365) (end 257.135 96.365) (width 1) (layer "F.Cu") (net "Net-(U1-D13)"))
 (segment (start 250.5 46.5) (end 246 42) (width 1) (layer "F.Cu") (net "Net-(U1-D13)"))
 (segment (start 239.24 94.9) (end 240.705 96.365) (width 1) (layer "F.Cu") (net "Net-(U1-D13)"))
 (segment (start 260.5 46.5) (end 250.5 46.5) (width 1) (layer "F.Cu") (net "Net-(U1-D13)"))
 (segment (start 195.6725 65) (end 254.5 65) (width 1) (layer "F.Cu") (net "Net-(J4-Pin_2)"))
 (segment (start 254.5 65) (end 258 68.5) (width 1) (layer "F.Cu") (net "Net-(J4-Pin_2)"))
 (segment (start 179.5 48.8275) (end 195.6725 65) (width 1) (layer "F.Cu") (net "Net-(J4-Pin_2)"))
 (segment (start 258 68.5) (end 258 91.38) (width 1) (layer "F.Cu") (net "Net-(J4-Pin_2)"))
 (segment (start 258 91.38) (end 254.48 94.9) (width 1) (layer "F.Cu") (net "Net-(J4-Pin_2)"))
 (segment (start 183 63) (end 222.58 63) (width 1) (layer "B.Cu") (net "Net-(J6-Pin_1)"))
 (segment (start 222.58 63) (end 229.08 69.5) (width 1) (layer "B.Cu") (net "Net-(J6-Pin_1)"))
 (segment (start 187.42 72.5) (end 218.46 72.5) (width 1) (layer "B.Cu") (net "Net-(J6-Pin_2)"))
 (segment (start 218.46 72.5) (end 221.46 69.5) (width 1) (layer "B.Cu") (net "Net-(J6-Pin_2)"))
 (segment (start 183 68.08) (end 187.42 72.5) (width 1) (layer "B.Cu") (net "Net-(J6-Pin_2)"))
 (segment (start 214.5 101) (end 220.44 101) (width 1) (layer "B.Cu") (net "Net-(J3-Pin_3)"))
 (segment (start 206.1725 92.6725) (end 214.5 101) (width 1) (layer "B.Cu") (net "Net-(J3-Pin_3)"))
 (segment (start 205.075 92.6725) (end 206.1725 92.6725) (width 1) (layer "B.Cu") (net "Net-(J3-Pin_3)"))
 (segment (start 220.44 101) (end 226.54 94.9) (width 1) (layer "B.Cu") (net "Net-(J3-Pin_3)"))
 (segment (start 211.235 58.5) (end 213.735 61) (width 1) (layer "F.Cu") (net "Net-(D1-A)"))
 (segment (start 208.81 58.5) (end 211.235 58.5) (width 1) (layer "F.Cu") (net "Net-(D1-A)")))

